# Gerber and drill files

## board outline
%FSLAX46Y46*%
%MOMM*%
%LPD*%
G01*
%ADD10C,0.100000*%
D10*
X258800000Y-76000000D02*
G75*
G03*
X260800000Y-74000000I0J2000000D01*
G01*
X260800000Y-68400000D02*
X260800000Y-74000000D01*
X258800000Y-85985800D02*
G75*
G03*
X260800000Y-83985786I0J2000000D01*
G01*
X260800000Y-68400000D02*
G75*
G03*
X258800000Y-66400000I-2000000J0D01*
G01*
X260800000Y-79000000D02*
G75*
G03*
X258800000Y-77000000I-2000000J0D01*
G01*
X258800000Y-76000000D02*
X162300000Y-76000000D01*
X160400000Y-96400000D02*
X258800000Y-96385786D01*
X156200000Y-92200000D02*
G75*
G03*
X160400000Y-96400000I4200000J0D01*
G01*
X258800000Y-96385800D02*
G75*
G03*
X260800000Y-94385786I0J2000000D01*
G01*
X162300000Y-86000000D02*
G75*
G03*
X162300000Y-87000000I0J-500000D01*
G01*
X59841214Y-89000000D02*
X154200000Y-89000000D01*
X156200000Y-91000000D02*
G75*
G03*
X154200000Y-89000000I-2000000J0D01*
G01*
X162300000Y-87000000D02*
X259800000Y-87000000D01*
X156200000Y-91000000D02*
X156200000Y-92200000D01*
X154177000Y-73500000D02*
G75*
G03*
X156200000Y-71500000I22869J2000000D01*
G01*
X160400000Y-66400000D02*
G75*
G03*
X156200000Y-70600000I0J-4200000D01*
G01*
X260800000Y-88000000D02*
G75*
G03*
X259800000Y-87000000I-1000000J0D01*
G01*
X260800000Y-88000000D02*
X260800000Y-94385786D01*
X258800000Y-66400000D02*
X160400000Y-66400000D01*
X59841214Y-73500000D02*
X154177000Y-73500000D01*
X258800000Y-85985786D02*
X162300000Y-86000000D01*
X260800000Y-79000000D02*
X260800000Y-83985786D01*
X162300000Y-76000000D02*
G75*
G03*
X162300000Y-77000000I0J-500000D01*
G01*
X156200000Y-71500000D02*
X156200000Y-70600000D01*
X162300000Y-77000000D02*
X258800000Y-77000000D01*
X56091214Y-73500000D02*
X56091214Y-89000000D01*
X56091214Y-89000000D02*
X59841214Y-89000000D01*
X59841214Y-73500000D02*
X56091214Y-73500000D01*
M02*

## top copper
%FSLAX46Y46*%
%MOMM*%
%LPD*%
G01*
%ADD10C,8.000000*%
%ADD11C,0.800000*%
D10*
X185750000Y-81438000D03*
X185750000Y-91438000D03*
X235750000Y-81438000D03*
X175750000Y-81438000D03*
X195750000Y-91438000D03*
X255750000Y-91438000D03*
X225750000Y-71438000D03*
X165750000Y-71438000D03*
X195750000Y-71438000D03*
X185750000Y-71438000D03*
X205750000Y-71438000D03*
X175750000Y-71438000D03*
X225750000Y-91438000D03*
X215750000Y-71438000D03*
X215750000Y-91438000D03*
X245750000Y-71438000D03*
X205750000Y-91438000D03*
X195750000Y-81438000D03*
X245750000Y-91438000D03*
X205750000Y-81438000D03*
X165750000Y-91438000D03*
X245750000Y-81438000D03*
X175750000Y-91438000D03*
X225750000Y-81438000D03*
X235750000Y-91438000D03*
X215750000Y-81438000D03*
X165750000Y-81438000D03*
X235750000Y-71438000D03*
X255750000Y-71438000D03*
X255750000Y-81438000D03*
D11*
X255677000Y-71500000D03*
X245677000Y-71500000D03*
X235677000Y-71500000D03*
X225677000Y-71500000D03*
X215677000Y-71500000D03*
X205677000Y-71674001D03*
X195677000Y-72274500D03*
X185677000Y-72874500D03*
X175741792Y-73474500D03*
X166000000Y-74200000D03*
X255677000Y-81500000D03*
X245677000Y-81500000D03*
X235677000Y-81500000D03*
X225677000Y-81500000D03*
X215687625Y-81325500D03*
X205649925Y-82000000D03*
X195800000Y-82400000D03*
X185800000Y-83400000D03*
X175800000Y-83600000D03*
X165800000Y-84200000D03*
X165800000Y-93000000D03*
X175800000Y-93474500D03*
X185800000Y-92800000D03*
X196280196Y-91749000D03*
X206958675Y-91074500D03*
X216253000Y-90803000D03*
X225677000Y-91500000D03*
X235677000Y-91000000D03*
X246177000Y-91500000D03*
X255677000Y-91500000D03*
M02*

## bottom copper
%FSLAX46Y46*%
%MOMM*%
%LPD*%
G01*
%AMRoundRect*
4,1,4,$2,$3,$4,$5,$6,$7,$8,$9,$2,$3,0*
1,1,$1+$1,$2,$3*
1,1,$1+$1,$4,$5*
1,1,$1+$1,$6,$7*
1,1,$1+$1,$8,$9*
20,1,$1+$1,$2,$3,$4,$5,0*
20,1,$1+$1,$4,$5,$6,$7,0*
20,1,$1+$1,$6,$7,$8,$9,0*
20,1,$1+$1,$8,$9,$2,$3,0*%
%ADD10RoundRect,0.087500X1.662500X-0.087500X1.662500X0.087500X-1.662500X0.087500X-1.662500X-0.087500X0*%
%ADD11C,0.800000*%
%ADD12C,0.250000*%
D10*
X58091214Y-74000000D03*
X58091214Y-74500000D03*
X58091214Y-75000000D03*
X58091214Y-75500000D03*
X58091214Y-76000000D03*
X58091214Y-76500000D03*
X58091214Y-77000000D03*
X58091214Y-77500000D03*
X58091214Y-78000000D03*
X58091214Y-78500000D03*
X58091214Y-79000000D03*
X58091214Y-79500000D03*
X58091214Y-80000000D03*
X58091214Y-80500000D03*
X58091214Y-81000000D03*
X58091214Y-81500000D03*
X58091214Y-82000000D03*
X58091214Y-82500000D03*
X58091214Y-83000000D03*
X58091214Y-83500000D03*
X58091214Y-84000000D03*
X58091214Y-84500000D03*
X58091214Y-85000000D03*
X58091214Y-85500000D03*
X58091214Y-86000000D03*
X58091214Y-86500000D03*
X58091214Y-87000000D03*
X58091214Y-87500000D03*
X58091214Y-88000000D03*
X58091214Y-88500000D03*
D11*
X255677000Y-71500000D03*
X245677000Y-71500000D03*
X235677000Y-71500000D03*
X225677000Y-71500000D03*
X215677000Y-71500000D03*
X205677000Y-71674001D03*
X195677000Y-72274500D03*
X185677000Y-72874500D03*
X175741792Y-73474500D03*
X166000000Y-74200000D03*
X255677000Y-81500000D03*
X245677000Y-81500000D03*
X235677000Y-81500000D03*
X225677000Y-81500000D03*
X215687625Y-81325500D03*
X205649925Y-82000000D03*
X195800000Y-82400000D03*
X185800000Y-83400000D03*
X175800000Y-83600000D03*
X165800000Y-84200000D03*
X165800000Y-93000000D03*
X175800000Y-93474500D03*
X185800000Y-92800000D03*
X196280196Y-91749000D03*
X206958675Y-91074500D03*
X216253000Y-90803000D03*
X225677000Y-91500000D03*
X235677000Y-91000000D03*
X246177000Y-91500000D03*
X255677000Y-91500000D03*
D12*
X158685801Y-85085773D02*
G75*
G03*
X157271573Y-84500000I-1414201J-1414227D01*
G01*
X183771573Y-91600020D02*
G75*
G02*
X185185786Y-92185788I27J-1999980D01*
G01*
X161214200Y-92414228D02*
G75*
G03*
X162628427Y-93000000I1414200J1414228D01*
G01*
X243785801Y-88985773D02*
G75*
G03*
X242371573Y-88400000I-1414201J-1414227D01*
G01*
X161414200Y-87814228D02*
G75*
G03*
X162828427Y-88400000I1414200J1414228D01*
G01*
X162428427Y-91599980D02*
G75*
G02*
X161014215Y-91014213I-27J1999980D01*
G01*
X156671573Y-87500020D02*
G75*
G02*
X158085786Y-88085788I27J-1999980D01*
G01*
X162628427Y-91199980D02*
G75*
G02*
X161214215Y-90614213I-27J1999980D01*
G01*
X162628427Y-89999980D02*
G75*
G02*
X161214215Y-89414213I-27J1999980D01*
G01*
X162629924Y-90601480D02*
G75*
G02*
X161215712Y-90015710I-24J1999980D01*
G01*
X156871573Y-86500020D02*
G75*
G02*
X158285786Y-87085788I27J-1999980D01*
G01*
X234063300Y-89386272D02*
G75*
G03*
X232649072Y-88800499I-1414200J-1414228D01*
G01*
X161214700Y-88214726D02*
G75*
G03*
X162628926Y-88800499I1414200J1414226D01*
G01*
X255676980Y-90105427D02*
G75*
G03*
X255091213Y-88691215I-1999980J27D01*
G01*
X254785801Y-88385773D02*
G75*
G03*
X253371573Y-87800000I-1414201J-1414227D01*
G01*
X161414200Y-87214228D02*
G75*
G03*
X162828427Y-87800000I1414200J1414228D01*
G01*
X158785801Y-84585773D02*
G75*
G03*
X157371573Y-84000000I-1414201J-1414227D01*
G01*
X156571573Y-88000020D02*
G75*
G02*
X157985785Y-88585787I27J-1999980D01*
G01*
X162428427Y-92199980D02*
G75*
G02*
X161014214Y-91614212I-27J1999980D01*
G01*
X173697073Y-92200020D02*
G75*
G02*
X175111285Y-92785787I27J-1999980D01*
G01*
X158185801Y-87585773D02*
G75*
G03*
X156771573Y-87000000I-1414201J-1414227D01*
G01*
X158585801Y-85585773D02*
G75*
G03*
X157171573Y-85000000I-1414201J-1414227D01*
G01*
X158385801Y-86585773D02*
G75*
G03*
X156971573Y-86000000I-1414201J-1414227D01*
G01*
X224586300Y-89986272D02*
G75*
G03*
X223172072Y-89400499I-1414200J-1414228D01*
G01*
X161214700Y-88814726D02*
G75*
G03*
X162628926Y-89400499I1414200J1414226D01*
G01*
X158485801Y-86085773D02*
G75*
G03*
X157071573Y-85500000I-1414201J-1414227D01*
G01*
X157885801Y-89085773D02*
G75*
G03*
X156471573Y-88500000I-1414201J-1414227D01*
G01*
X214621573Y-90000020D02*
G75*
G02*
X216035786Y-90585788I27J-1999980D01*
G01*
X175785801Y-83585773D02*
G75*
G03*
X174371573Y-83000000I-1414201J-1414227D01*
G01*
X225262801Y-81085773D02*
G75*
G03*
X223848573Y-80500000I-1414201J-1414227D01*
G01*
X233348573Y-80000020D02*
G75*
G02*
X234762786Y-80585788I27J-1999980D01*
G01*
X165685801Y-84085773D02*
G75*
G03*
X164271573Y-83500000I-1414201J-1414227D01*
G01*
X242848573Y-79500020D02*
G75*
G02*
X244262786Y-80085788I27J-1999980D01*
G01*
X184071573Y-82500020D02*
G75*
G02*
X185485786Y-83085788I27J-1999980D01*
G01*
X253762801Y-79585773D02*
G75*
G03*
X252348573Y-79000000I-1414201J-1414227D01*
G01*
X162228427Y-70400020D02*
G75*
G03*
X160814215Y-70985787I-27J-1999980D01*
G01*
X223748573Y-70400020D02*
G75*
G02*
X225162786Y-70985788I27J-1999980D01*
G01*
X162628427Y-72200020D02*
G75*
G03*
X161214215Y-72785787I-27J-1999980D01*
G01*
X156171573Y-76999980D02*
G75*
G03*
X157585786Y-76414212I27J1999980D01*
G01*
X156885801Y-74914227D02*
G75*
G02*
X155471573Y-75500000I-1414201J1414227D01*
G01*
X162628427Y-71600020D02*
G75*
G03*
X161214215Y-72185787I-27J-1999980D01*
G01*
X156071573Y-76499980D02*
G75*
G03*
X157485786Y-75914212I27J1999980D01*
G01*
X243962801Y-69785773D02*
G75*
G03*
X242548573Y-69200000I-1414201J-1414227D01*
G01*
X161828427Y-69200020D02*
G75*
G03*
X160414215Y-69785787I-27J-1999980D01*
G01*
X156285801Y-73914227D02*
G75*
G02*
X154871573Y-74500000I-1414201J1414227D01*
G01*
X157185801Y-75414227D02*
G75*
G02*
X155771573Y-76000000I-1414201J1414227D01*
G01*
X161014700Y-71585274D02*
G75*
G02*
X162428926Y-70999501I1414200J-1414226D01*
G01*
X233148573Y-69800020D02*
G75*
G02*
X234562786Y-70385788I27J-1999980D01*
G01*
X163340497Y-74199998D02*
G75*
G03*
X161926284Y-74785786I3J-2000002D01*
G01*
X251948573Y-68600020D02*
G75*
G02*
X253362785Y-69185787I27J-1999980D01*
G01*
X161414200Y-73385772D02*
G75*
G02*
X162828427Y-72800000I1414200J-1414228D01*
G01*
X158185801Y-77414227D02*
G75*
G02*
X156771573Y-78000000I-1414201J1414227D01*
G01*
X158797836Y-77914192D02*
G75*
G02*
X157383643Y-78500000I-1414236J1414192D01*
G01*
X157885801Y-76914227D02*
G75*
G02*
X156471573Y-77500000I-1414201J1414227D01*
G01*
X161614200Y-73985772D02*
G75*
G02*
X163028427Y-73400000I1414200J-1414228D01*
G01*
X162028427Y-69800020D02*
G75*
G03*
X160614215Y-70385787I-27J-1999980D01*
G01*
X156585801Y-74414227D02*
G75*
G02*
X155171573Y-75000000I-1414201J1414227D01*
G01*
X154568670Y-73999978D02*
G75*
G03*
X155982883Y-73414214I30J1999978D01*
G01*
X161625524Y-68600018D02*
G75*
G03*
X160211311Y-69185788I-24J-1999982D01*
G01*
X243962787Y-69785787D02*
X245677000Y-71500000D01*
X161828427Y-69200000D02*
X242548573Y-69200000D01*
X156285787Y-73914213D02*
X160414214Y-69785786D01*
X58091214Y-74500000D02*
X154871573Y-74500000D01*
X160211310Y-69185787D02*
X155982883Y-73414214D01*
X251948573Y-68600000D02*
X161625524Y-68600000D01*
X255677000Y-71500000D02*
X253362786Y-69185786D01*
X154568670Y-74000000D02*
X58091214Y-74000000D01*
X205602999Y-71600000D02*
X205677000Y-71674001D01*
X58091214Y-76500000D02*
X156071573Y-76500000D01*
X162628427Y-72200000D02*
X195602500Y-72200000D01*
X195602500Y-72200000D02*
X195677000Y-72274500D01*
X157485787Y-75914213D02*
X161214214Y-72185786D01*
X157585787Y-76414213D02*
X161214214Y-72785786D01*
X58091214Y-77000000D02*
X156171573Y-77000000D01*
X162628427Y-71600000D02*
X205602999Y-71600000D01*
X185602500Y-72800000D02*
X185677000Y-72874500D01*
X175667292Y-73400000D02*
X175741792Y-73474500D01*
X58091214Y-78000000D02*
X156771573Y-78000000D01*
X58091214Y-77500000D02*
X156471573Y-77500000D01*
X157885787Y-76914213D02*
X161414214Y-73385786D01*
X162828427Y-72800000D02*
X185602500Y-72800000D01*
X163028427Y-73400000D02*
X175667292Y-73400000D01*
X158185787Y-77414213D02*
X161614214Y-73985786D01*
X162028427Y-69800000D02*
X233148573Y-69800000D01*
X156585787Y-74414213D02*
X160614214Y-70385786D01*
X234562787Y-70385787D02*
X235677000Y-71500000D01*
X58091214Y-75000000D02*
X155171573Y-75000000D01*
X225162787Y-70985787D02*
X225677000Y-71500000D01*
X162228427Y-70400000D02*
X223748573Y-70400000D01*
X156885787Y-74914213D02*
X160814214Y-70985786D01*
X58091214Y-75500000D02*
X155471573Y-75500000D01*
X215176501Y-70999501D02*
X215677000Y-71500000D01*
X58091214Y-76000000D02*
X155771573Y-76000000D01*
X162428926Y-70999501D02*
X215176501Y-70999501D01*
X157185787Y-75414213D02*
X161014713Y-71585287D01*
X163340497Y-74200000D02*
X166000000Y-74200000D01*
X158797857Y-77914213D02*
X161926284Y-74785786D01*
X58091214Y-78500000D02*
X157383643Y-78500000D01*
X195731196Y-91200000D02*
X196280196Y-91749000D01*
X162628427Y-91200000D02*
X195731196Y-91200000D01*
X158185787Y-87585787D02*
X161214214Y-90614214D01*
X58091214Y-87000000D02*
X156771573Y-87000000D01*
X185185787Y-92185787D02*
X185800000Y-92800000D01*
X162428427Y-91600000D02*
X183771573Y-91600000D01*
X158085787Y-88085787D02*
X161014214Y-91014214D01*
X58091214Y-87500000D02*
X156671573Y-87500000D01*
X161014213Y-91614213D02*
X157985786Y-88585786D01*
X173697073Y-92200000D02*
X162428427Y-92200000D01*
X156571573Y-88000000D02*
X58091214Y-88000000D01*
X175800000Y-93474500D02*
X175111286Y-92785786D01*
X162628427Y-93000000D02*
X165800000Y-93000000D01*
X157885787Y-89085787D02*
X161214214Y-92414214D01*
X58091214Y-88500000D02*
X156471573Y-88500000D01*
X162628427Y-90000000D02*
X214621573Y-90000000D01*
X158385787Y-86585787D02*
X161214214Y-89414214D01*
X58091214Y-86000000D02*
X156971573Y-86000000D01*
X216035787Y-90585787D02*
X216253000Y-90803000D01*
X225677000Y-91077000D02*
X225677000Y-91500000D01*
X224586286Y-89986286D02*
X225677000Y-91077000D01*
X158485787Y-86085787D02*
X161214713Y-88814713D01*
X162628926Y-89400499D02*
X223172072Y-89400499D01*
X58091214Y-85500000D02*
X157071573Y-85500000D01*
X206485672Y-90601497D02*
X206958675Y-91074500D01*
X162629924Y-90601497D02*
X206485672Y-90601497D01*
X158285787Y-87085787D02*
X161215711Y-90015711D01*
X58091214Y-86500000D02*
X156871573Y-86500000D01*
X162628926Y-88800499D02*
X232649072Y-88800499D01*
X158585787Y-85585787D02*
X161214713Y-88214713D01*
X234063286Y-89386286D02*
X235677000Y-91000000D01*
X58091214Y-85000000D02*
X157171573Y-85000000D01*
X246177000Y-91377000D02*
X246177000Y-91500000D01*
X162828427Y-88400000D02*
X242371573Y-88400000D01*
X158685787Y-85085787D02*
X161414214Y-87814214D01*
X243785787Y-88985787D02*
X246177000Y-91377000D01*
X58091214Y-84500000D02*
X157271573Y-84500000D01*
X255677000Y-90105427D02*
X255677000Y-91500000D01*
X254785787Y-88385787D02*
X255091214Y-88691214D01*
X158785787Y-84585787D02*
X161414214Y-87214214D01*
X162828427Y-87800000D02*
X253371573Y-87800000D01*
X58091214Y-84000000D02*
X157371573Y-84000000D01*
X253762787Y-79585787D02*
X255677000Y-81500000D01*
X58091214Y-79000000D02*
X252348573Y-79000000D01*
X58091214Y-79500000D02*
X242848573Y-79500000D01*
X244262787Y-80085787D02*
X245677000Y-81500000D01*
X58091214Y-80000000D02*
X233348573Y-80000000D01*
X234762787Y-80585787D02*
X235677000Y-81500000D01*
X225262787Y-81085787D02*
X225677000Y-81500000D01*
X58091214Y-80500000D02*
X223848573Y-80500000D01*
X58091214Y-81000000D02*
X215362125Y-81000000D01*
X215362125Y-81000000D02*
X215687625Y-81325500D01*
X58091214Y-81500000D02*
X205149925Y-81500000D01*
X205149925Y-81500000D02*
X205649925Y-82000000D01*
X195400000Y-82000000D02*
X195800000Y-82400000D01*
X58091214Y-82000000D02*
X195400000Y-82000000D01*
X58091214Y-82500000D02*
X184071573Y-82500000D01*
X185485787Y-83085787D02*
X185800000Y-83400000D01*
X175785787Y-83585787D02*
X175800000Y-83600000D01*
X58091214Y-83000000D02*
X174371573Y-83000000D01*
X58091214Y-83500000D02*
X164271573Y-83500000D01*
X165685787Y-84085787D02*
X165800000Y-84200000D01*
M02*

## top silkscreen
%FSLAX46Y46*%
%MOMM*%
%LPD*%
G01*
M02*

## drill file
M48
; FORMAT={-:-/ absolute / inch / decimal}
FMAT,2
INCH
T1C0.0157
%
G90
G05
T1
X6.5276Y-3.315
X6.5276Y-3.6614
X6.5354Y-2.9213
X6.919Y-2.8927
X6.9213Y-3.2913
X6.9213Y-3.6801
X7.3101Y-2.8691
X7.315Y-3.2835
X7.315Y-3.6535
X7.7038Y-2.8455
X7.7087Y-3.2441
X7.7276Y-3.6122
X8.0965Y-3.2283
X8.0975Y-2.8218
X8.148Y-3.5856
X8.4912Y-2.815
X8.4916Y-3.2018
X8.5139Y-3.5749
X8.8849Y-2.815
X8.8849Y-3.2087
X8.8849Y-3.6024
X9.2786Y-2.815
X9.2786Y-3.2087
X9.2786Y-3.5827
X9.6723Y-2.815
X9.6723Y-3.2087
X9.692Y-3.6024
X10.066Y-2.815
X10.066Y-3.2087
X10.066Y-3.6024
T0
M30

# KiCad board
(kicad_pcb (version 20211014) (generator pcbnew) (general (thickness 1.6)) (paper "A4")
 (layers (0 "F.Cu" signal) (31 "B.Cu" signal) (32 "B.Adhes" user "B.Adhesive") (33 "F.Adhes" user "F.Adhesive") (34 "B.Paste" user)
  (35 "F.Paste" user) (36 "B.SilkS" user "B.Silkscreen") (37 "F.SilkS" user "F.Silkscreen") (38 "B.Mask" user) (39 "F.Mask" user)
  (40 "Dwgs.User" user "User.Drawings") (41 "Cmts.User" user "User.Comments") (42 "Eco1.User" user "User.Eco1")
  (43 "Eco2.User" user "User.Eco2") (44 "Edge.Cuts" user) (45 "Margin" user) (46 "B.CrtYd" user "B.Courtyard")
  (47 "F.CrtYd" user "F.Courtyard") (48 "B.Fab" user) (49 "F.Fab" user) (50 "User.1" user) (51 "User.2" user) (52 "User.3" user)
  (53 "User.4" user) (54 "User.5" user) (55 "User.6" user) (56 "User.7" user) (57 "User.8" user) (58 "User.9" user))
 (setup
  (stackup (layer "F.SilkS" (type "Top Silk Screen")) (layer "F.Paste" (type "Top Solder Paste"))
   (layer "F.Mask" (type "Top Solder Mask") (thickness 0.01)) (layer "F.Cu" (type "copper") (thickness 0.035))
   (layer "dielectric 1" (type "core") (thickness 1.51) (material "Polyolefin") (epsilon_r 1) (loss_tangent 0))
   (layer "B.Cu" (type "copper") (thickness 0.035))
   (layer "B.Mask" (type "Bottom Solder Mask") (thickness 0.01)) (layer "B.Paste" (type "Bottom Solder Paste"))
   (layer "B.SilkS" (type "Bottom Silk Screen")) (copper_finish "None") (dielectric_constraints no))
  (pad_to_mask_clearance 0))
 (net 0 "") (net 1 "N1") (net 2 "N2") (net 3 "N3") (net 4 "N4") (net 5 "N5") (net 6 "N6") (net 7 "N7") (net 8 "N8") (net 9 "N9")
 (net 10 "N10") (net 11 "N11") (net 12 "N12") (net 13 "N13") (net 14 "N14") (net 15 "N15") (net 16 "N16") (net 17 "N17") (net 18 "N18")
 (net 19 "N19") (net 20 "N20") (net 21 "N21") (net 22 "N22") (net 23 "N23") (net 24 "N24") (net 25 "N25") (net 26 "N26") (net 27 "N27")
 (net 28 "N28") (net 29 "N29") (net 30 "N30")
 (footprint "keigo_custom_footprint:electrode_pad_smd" (layer "F.Cu") (at 185.75 81.438)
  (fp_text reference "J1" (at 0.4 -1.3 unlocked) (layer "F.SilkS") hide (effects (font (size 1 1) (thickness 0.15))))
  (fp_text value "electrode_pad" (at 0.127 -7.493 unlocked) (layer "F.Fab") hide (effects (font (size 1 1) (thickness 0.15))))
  (pad "" smd circle (at 0 0) (size 8 8) (layers "F.Cu" "F.Mask") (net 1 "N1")))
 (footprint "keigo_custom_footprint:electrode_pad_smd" (layer "F.Cu") (at 185.75 91.438)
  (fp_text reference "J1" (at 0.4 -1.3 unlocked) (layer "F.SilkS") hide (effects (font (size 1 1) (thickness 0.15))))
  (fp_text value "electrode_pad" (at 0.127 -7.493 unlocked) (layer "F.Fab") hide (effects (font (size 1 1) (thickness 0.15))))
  (pad "" smd circle (at 0 0) (size 8 8) (layers "F.Cu" "F.Mask") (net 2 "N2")))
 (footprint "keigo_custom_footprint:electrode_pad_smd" (layer "F.Cu") (at 235.75 81.438)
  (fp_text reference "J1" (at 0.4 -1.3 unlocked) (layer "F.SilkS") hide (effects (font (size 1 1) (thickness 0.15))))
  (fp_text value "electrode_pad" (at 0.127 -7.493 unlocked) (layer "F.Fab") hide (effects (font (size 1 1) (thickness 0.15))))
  (pad "" smd circle (at 0 0) (size 8 8) (layers "F.Cu" "F.Mask") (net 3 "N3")))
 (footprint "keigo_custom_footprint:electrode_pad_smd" (layer "F.Cu") (at 175.75 81.438)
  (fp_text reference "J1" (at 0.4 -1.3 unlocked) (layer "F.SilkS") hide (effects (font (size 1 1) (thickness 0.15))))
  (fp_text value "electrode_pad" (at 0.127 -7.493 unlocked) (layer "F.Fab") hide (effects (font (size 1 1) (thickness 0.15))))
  (pad "" smd circle (at 0 0) (size 8 8) (layers "F.Cu" "F.Mask") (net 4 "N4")))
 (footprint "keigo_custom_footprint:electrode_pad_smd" (layer "F.Cu") (at 195.75 91.438)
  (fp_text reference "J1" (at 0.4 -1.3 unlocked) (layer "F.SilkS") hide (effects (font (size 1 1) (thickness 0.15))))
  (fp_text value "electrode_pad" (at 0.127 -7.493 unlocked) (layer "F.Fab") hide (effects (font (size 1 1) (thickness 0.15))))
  (pad "" smd circle (at 0 0) (size 8 8) (layers "F.Cu" "F.Mask") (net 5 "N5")))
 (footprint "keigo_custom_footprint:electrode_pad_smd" (layer "F.Cu") (at 255.75 91.438)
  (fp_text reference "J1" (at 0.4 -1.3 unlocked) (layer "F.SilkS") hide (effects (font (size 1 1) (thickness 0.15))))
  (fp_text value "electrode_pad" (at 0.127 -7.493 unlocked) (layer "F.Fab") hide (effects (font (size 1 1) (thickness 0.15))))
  (pad "21" smd circle (at 0 0) (size 8 8) (layers "F.Cu" "F.Mask") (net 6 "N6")))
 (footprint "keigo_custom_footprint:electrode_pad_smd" (layer "F.Cu") (at 225.75 71.438)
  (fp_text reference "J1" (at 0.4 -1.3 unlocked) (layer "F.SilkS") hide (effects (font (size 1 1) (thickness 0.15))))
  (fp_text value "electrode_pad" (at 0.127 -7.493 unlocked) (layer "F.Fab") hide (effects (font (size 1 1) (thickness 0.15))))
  (pad "" smd circle (at 0 0) (size 8 8) (layers "F.Cu" "F.Mask") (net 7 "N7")))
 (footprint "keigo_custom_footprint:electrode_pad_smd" (layer "F.Cu") (at 165.75 71.438)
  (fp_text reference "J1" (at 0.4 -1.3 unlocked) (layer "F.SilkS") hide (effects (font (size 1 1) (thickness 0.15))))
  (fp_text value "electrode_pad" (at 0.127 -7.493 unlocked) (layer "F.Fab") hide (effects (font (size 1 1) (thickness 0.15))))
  (pad "10" smd circle (at 0 0) (size 8 8) (layers "F.Cu" "F.Mask") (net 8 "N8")))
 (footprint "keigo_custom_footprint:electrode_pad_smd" (layer "F.Cu") (at 195.75 71.438)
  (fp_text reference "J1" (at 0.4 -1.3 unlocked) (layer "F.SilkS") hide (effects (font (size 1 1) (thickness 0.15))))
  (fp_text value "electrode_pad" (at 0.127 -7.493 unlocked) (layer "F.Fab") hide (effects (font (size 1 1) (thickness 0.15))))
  (pad "" smd circle (at 0 0) (size 8 8) (layers "F.Cu" "F.Mask") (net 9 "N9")))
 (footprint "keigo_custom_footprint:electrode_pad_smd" (layer "F.Cu") (at 185.75 71.438)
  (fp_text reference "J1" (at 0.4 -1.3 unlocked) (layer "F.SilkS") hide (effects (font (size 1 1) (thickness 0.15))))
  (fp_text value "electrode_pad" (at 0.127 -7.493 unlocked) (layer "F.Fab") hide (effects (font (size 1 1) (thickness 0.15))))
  (pad "" smd circle (at 0 0) (size 8 8) (layers "F.Cu" "F.Mask") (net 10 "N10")))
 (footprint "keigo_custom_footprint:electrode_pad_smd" (layer "F.Cu") (at 205.75 71.438)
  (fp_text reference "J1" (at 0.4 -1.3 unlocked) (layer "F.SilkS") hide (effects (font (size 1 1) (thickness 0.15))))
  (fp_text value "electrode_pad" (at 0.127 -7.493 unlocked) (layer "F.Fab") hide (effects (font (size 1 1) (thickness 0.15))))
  (pad "" smd circle (at 0 0) (size 8 8) (layers "F.Cu" "F.Mask") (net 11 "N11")))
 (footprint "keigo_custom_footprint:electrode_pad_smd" (layer "F.Cu") (at 175.75 71.438)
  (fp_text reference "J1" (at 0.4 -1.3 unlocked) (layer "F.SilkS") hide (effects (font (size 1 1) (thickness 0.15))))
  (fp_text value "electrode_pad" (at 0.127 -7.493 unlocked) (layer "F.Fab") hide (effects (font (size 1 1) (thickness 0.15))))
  (pad "9" smd circle (at 0 0) (size 8 8) (layers "F.Cu" "F.Mask") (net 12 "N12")))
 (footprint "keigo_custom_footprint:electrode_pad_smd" (layer "F.Cu") (at 225.75 91.438)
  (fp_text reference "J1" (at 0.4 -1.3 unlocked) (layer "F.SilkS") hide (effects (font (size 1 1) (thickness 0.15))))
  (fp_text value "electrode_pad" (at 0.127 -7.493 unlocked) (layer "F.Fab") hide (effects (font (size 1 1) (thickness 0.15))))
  (pad "" smd circle (at 0 0) (size 8 8) (layers "F.Cu" "F.Mask") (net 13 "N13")))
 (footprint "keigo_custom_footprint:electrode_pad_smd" (layer "F.Cu") (at 215.75 71.438)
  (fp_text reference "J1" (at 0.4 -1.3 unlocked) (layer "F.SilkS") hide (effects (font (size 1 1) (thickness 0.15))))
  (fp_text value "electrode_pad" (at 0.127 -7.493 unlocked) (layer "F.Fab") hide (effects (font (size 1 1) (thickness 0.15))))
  (pad "" smd circle (at 0 0) (size 8 8) (layers "F.Cu" "F.Mask") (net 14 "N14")))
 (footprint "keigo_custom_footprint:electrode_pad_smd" (layer "F.Cu") (at 215.75 91.438)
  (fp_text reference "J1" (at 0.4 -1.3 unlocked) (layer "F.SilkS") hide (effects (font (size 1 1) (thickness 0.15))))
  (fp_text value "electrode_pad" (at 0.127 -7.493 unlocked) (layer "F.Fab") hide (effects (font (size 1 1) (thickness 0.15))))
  (pad "" smd circle (at 0 0) (size 8 8) (layers "F.Cu" "F.Mask") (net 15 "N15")))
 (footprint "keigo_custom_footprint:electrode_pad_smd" (layer "F.Cu") (at 245.75 71.438)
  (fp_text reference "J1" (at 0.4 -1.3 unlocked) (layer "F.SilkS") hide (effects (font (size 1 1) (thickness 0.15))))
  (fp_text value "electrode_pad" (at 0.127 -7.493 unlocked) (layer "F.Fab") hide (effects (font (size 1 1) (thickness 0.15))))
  (pad "" smd circle (at 0 0) (size 8 8) (layers "F.Cu" "F.Mask") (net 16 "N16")))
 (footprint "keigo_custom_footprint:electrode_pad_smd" (layer "F.Cu") (at 205.75 91.438)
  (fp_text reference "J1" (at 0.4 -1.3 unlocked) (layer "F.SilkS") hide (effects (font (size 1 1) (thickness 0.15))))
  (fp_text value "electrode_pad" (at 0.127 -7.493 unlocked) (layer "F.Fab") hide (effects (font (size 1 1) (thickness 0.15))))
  (pad "" smd circle (at 0 0) (size 8 8) (layers "F.Cu" "F.Mask") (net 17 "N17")))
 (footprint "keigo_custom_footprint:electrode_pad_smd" (layer "F.Cu") (at 195.75 81.438)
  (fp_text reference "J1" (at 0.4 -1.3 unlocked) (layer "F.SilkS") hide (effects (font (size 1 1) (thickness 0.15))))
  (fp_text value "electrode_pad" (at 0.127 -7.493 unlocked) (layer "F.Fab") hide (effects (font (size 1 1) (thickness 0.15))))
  (pad "" smd circle (at 0 0) (size 8 8) (layers "F.Cu" "F.Mask") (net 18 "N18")))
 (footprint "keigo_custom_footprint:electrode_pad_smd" (layer "F.Cu") (at 245.75 91.438)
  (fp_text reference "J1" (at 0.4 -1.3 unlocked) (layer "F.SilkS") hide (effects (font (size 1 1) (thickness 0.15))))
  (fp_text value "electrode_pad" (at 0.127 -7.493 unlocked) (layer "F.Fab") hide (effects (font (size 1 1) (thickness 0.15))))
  (pad "" smd circle (at 0 0) (size 8 8) (layers "F.Cu" "F.Mask") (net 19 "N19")))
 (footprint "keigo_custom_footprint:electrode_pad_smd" (layer "F.Cu") (at 205.75 81.438)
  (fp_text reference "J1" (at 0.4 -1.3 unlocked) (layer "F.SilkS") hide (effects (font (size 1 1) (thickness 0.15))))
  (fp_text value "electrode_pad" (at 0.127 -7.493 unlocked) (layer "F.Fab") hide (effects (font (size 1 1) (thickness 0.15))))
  (pad "" smd circle (at 0 0) (size 8 8) (layers "F.Cu" "F.Mask") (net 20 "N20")))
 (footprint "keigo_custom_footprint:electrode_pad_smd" (layer "F.Cu") (at 165.75 91.438)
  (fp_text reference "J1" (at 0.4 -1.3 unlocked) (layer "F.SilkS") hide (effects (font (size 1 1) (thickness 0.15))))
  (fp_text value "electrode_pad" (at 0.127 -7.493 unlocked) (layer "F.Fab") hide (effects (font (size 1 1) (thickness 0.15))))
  (pad "30" smd circle (at 0 0) (size 8 8) (layers "F.Cu" "F.Mask") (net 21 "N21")))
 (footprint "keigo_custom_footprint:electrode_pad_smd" (layer "F.Cu") (at 245.75 81.438)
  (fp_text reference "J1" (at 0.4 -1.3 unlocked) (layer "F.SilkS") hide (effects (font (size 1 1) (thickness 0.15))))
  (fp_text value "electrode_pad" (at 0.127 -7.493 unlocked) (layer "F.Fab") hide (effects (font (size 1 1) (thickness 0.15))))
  (pad "" smd circle (at 0 0) (size 8 8) (layers "F.Cu" "F.Mask") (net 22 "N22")))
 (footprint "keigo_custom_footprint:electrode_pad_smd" (layer "F.Cu") (at 175.75 91.438)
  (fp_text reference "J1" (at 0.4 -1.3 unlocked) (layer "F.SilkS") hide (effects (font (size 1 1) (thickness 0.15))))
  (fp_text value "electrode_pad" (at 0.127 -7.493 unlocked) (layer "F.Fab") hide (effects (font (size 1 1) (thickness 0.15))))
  (pad "" smd circle (at 0 0) (size 8 8) (layers "F.Cu" "F.Mask") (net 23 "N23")))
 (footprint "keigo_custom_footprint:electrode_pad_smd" (layer "F.Cu") (at 225.75 81.438)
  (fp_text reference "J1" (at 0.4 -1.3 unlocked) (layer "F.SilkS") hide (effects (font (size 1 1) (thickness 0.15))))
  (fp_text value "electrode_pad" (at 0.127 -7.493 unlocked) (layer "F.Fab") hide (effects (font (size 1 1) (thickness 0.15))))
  (pad "" smd circle (at 0 0) (size 8 8) (layers "F.Cu" "F.Mask") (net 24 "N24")))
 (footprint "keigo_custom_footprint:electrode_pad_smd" (layer "F.Cu") (at 235.75 91.438)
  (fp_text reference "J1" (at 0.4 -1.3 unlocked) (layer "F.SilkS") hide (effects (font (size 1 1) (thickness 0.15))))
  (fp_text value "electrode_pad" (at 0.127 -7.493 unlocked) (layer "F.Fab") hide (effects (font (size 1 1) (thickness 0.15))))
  (pad "" smd circle (at 0 0) (size 8 8) (layers "F.Cu" "F.Mask") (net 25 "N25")))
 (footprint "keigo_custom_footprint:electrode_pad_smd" (layer "F.Cu") (at 215.75 81.438)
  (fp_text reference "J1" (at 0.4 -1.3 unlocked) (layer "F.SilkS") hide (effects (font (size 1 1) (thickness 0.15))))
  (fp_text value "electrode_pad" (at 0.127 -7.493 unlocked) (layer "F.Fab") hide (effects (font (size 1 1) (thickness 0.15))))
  (pad "" smd circle (at 0 0) (size 8 8) (layers "F.Cu" "F.Mask") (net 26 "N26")))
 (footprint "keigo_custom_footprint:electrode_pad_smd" (layer "F.Cu") (at 165.75 81.438)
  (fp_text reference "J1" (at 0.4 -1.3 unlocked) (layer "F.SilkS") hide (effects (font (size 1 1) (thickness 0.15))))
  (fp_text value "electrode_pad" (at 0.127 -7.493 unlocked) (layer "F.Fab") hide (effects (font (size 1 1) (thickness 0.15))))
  (pad "20" smd circle (at 0 0) (size 8 8) (layers "F.Cu" "F.Mask") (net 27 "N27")))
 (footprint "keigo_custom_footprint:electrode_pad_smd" (layer "F.Cu") (at 235.75 71.438)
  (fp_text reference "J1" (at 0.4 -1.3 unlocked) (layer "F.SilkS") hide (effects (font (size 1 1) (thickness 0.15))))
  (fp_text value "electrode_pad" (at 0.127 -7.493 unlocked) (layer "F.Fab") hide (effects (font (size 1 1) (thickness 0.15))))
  (pad "" smd circle (at 0 0) (size 8 8) (layers "F.Cu" "F.Mask") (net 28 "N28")))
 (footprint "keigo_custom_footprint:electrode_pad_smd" (layer "F.Cu") (at 255.75 71.438)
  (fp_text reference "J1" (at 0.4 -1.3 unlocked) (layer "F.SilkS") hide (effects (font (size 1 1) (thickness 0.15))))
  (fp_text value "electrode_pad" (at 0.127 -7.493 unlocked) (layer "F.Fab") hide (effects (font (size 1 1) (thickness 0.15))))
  (pad "1" smd circle (at 0 0) (size 8 8) (layers "F.Cu" "F.Mask") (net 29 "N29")))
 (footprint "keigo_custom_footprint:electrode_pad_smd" (layer "F.Cu") (at 255.75 81.438)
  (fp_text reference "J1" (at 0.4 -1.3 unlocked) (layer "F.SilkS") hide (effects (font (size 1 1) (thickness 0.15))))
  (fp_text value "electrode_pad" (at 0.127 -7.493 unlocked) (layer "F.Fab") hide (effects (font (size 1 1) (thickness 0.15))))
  (pad "11" smd circle (at 0 0) (size 8 8) (layers "F.Cu" "F.Mask") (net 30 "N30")))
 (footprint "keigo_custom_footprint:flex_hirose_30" (layer "B.Cu") (at 58.091214 80.75 -90)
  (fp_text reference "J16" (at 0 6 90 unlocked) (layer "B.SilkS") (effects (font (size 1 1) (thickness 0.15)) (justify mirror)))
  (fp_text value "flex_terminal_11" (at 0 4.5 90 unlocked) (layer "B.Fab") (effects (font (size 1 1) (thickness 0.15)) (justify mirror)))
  (fp_line (start -7.25 2) (end 8.25 2) (layer "Edge.Cuts") (width 0.1))
  (fp_line (start 8.25 2) (end 8.25 -1.75) (layer "Edge.Cuts") (width 0.1))
  (fp_line (start -7.25 -1.75) (end -7.25 2) (layer "Edge.Cuts") (width 0.1))
  (pad "1" smd roundrect (at -6.75 0 90) (size 0.35 3.5) (layers "B.Cu" "B.Paste" "B.Mask") (roundrect_rratio 0.25) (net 29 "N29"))
  (pad "2" smd roundrect (at -6.25 0 90) (size 0.35 3.5) (layers "B.Cu" "B.Paste" "B.Mask") (roundrect_rratio 0.25) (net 16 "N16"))
  (pad "3" smd roundrect (at -5.75 0 90) (size 0.35 3.5) (layers "B.Cu" "B.Paste" "B.Mask") (roundrect_rratio 0.25) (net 28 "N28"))
  (pad "4" smd roundrect (at -5.25 0 90) (size 0.35 3.5) (layers "B.Cu" "B.Paste" "B.Mask") (roundrect_rratio 0.25) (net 7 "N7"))
  (pad "5" smd roundrect (at -4.75 0 90) (size 0.35 3.5) (layers "B.Cu" "B.Paste" "B.Mask") (roundrect_rratio 0.25) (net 14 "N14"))
  (pad "6" smd roundrect (at -4.25 0 90) (size 0.35 3.5) (layers "B.Cu" "B.Paste" "B.Mask") (roundrect_rratio 0.25) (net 11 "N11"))
  (pad "7" smd roundrect (at -3.75 0 90) (size 0.35 3.5) (layers "B.Cu" "B.Paste" "B.Mask") (roundrect_rratio 0.25) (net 9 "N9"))
  (pad "8" smd roundrect (at -3.25 0 90) (size 0.35 3.5) (layers "B.Cu" "B.Paste" "B.Mask") (roundrect_rratio 0.25) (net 10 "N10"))
  (pad "9" smd roundrect (at -2.75 0 90) (size 0.35 3.5) (layers "B.Cu" "B.Paste" "B.Mask") (roundrect_rratio 0.25) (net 12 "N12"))
  (pad "10" smd roundrect (at -2.25 0 90) (size 0.35 3.5) (layers "B.Cu" "B.Paste" "B.Mask") (roundrect_rratio 0.25) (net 8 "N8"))
  (pad "11" smd roundrect (at -1.75 0 90) (size 0.35 3.5) (layers "B.Cu" "B.Paste" "B.Mask") (roundrect_rratio 0.25) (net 30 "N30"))
  (pad "12" smd roundrect (at -1.25 0 90) (size 0.35 3.5) (layers "B.Cu" "B.Paste" "B.Mask") (roundrect_rratio 0.25) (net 22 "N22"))
  (pad "13" smd roundrect (at -0.75 0 90) (size 0.35 3.5) (layers "B.Cu" "B.Paste" "B.Mask") (roundrect_rratio 0.25) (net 3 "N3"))
  (pad "14" smd roundrect (at -0.25 0 90) (size 0.35 3.5) (layers "B.Cu" "B.Paste" "B.Mask") (roundrect_rratio 0.25) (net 24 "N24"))
  (pad "15" smd roundrect (at 0.25 0 90) (size 0.35 3.5) (layers "B.Cu" "B.Paste" "B.Mask") (roundrect_rratio 0.25) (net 26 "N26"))
  (pad "16" smd roundrect (at 0.75 0 90) (size 0.35 3.5) (layers "B.Cu" "B.Paste" "B.Mask") (roundrect_rratio 0.25) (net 20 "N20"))
  (pad "17" smd roundrect (at 1.25 0 90) (size 0.35 3.5) (layers "B.Cu" "B.Paste" "B.Mask") (roundrect_rratio 0.25) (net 18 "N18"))
  (pad "18" smd roundrect (at 1.75 0 90) (size 0.35 3.5) (layers "B.Cu" "B.Paste" "B.Mask") (roundrect_rratio 0.25) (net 1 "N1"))
  (pad "19" smd roundrect (at 2.25 0 90) (size 0.35 3.5) (layers "B.Cu" "B.Paste" "B.Mask") (roundrect_rratio 0.25) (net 4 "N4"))
  (pad "20" smd roundrect (at 2.75 0 90) (size 0.35 3.5) (layers "B.Cu" "B.Paste" "B.Mask") (roundrect_rratio 0.25) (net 27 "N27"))
  (pad "21" smd roundrect (at 3.25 0 90) (size 0.35 3.5) (layers "B.Cu" "B.Paste" "B.Mask") (roundrect_rratio 0.25) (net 6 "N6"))
  (pad "22" smd roundrect (at 3.75 0 90) (size 0.35 3.5) (layers "B.Cu" "B.Paste" "B.Mask") (roundrect_rratio 0.25) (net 19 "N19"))
  (pad "23" smd roundrect (at 4.25 0 90) (size 0.35 3.5) (layers "B.Cu" "B.Paste" "B.Mask") (roundrect_rratio 0.25) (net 25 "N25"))
  (pad "24" smd roundrect (at 4.75 0 90) (size 0.35 3.5) (layers "B.Cu" "B.Paste" "B.Mask") (roundrect_rratio 0.25) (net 13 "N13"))
  (pad "25" smd roundrect (at 5.25 0 90) (size 0.35 3.5) (layers "B.Cu" "B.Paste" "B.Mask") (roundrect_rratio 0.25) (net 15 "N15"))
  (pad "26" smd roundrect (at 5.75 0 90) (size 0.35 3.5) (layers "B.Cu" "B.Paste" "B.Mask") (roundrect_rratio 0.25) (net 17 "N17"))
  (pad "27" smd roundrect (at 6.25 0 90) (size 0.35 3.5) (layers "B.Cu" "B.Paste" "B.Mask") (roundrect_rratio 0.25) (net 5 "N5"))
  (pad "28" smd roundrect (at 6.75 0 90) (size 0.35 3.5) (layers "B.Cu" "B.Paste" "B.Mask") (roundrect_rratio 0.25) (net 2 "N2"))
  (pad "29" smd roundrect (at 7.25 0 90) (size 0.35 3.5) (layers "B.Cu" "B.Paste" "B.Mask") (roundrect_rratio 0.25) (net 23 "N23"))
  (pad "30" smd roundrect (at 7.75 0 90) (size 0.35 3.5) (layers "B.Cu" "B.Paste" "B.Mask") (roundrect_rratio 0.25) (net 21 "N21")))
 (gr_arc (start 260.8 74) (mid 260.214214 75.414214) (end 258.8 76) (layer "Edge.Cuts") (width 0.1))
 (gr_line (start 260.8 68.4) (end 260.8 74) (layer "Edge.Cuts") (width 0.1))
 (gr_arc (start 260.8 83.985786) (mid 260.214214 85.4) (end 258.8 85.985786) (layer "Edge.Cuts") (width 0.1))
 (gr_arc (start 258.8 66.4) (mid 260.214214 66.985786) (end 260.8 68.4) (layer "Edge.Cuts") (width 0.1))
 (gr_arc (start 258.8 77) (mid 260.214214 77.585786) (end 260.8 79) (layer "Edge.Cuts") (width 0.1))
 (gr_line (start 258.8 76) (end 162.3 76) (layer "Edge.Cuts") (width 0.1))
 (gr_line (start 160.4 96.4) (end 258.8 96.385786) (layer "Edge.Cuts") (width 0.1))
 (gr_arc (start 160.4 96.4) (mid 157.430152 95.169848) (end 156.2 92.2) (layer "Edge.Cuts") (width 0.1))
 (gr_arc (start 260.8 94.385786) (mid 260.214214 95.8) (end 258.8 96.385786) (layer "Edge.Cuts") (width 0.1))
 (gr_arc (start 162.3 87) (mid 161.8 86.5) (end 162.3 86) (layer "Edge.Cuts") (width 0.1))
 (gr_line (start 59.841214 89) (end 154.2 89) (layer "Edge.Cuts") (width 0.1))
 (gr_arc (start 154.2 89) (mid 155.614214 89.585786) (end 156.2 91) (layer "Edge.Cuts") (width 0.1))
 (gr_line (start 162.3 87) (end 259.8 87) (layer "Edge.Cuts") (width 0.1))
 (gr_line (start 156.2 91) (end 156.2 92.2) (layer "Edge.Cuts") (width 0.1))
 (gr_arc (start 156.2 71.5) (mid 155.606067 72.922369) (end 154.177 73.5) (layer "Edge.Cuts") (width 0.1))
 (gr_arc (start 156.2 70.6) (mid 157.430152 67.630152) (end 160.4 66.4) (layer "Edge.Cuts") (width 0.1))
 (gr_arc (start 259.8 87) (mid 260.507107 87.292893) (end 260.8 88) (layer "Edge.Cuts") (width 0.1))
 (gr_line (start 260.8 88) (end 260.8 94.385786) (layer "Edge.Cuts") (width 0.1))
 (gr_line (start 258.8 66.4) (end 160.4 66.4) (layer "Edge.Cuts") (width 0.1))
 (gr_line (start 59.841214 73.5) (end 154.177 73.5) (layer "Edge.Cuts") (width 0.1))
 (gr_line (start 258.8 85.985786) (end 162.3 86) (layer "Edge.Cuts") (width 0.1))
 (gr_line (start 260.8 79) (end 260.8 83.985786) (layer "Edge.Cuts") (width 0.1))
 (gr_arc (start 162.3 77) (mid 161.8 76.5) (end 162.3 76) (layer "Edge.Cuts") (width 0.1))
 (gr_line (start 156.2 71.5) (end 156.2 70.6) (layer "Edge.Cuts") (width 0.1))
 (gr_line (start 162.3 77) (end 258.8 77) (layer "Edge.Cuts") (width 0.1))
 (via (at 255.677 71.5) (size 0.8) (drill 0.4) (layers "F.Cu" "B.Cu") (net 29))
 (segment (start 251.948573 68.6) (end 161.625524 68.6) (width 0.25) (layer "B.Cu") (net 29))
 (segment (start 160.21131 69.185787) (end 155.982883 73.414214) (width 0.25) (layer "B.Cu") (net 29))
 (segment (start 255.677 71.5) (end 253.362786 69.185786) (width 0.25) (layer "B.Cu") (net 29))
 (segment (start 154.56867 74) (end 58.091214 74) (width 0.25) (layer "B.Cu") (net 29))
 (arc (start 253.362786 69.185786) (mid 252.71394 68.752241) (end 251.948573 68.6) (width 0.25) (layer "B.Cu") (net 29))
 (arc (start 155.982883 73.414214) (mid 155.334037 73.847759) (end 154.56867 74) (width 0.25) (layer "B.Cu") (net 29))
 (arc (start 160.21131 69.185787) (mid 160.860157 68.752241) (end 161.625524 68.6) (width 0.25) (layer "B.Cu") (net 29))
 (via (at 245.677 71.5) (size 0.8) (drill 0.4) (layers "F.Cu" "B.Cu") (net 16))
 (segment (start 58.091214 74.5) (end 154.871573 74.5) (width 0.25) (layer "B.Cu") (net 16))
 (segment (start 161.828427 69.2) (end 242.548573 69.2) (width 0.25) (layer "B.Cu") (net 16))
 (segment (start 156.285787 73.914213) (end 160.414214 69.785786) (width 0.25) (layer "B.Cu") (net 16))
 (segment (start 243.962787 69.785787) (end 245.677 71.5) (width 0.25) (layer "B.Cu") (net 16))
 (arc (start 154.871573 74.5) (mid 155.63694 74.347759) (end 156.285787 73.914213) (width 0.25) (layer "B.Cu") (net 16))
 (arc (start 242.548573 69.2) (mid 243.31394 69.352241) (end 243.962787 69.785787) (width 0.25) (layer "B.Cu") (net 16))
 (arc (start 160.414214 69.785786) (mid 161.06306 69.352241) (end 161.828427 69.2) (width 0.25) (layer "B.Cu") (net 16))
 (via (at 235.677 71.5) (size 0.8) (drill 0.4) (layers "F.Cu" "B.Cu") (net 28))
 (segment (start 156.585787 74.414213) (end 160.614214 70.385786) (width 0.25) (layer "B.Cu") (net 28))
 (segment (start 162.028427 69.8) (end 233.148573 69.8) (width 0.25) (layer "B.Cu") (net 28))
 (segment (start 58.091214 75) (end 155.171573 75) (width 0.25) (layer "B.Cu") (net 28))
 (segment (start 234.562787 70.385787) (end 235.677 71.5) (width 0.25) (layer "B.Cu") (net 28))
 (arc (start 155.171573 75) (mid 155.93694 74.847759) (end 156.585787 74.414213) (width 0.25) (layer "B.Cu") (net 28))
 (arc (start 234.562787 70.385787) (mid 233.91394 69.952241) (end 233.148573 69.8) (width 0.25) (layer "B.Cu") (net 28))
 (arc (start 160.614214 70.385786) (mid 161.26306 69.952241) (end 162.028427 69.8) (width 0.25) (layer "B.Cu") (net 28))
 (via (at 225.677 71.5) (size 0.8) (drill 0.4) (layers "F.Cu" "B.Cu") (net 7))
 (segment (start 162.228427 70.4) (end 223.748573 70.4) (width 0.25) (layer "B.Cu") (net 7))
 (segment (start 58.091214 75.5) (end 155.471573 75.5) (width 0.25) (layer "B.Cu") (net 7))
 (segment (start 225.162787 70.985787) (end 225.677 71.5) (width 0.25) (layer "B.Cu") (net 7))
 (segment (start 156.885787 74.914213) (end 160.814214 70.985786) (width 0.25) (layer "B.Cu") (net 7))
 (arc (start 225.162787 70.985787) (mid 224.51394 70.552241) (end 223.748573 70.4) (width 0.25) (layer "B.Cu") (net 7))
 (arc (start 160.814214 70.985786) (mid 161.46306 70.552241) (end 162.228427 70.4) (width 0.25) (layer "B.Cu") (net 7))
 (arc (start 155.471573 75.5) (mid 156.23694 75.347759) (end 156.885787 74.914213) (width 0.25) (layer "B.Cu") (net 7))
 (via (at 215.677 71.5) (size 0.8) (drill 0.4) (layers "F.Cu" "B.Cu") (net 14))
 (segment (start 215.176501 70.999501) (end 215.677 71.5) (width 0.25) (layer "B.Cu") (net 14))
 (segment (start 58.091214 76) (end 155.771573 76) (width 0.25) (layer "B.Cu") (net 14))
 (segment (start 162.428926 70.999501) (end 215.176501 70.999501) (width 0.25) (layer "B.Cu") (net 14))
 (segment (start 157.185787 75.414213) (end 161.014713 71.585287) (width 0.25) (layer "B.Cu") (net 14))
 (arc (start 155.771573 76) (mid 156.53694 75.847759) (end 157.185787 75.414213) (width 0.25) (layer "B.Cu") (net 14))
 (arc (start 162.428926 70.999501) (mid 161.663559 71.151742) (end 161.014713 71.585287) (width 0.25) (layer "B.Cu") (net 14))
 (via (at 205.677 71.674001) (size 0.8) (drill 0.4) (layers "F.Cu" "B.Cu") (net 11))
 (segment (start 157.485787 75.914213) (end 161.214214 72.185786) (width 0.25) (layer "B.Cu") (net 11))
 (segment (start 162.628427 71.6) (end 205.602999 71.6) (width 0.25) (layer "B.Cu") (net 11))
 (segment (start 58.091214 76.5) (end 156.071573 76.5) (width 0.25) (layer "B.Cu") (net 11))
 (segment (start 205.602999 71.6) (end 205.677 71.674001) (width 0.25) (layer "B.Cu") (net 11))
 (arc (start 157.485787 75.914213) (mid 156.83694 76.347759) (end 156.071573 76.5) (width 0.25) (layer "B.Cu") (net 11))
 (arc (start 161.214214 72.185786) (mid 161.86306 71.752241) (end 162.628427 71.6) (width 0.25) (layer "B.Cu") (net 11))
 (via (at 195.677 72.2745) (size 0.8) (drill 0.4) (layers "F.Cu" "B.Cu") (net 9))
 (segment (start 157.585787 76.414213) (end 161.214214 72.785786) (width 0.25) (layer "B.Cu") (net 9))
 (segment (start 162.628427 72.2) (end 195.6025 72.2) (width 0.25) (layer "B.Cu") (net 9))
 (segment (start 58.091214 77) (end 156.171573 77) (width 0.25) (layer "B.Cu") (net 9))
 (segment (start 195.6025 72.2) (end 195.677 72.2745) (width 0.25) (layer "B.Cu") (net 9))
 (arc (start 161.214214 72.785786) (mid 161.86306 72.352241) (end 162.628427 72.2) (width 0.25) (layer "B.Cu") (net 9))
 (arc (start 157.585787 76.414213) (mid 156.93694 76.847759) (end 156.171573 77) (width 0.25) (layer "B.Cu") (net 9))
 (via (at 185.677 72.8745) (size 0.8) (drill 0.4) (layers "F.Cu" "B.Cu") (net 10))
 (segment (start 58.091214 77.5) (end 156.471573 77.5) (width 0.25) (layer "B.Cu") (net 10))
 (segment (start 157.885787 76.914213) (end 161.414214 73.385786) (width 0.25) (layer "B.Cu") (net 10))
 (segment (start 162.828427 72.8) (end 185.6025 72.8) (width 0.25) (layer "B.Cu") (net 10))
 (segment (start 185.6025 72.8) (end 185.677 72.8745) (width 0.25) (layer "B.Cu") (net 10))
 (arc (start 156.471573 77.5) (mid 157.23694 77.347759) (end 157.885787 76.914213) (width 0.25) (layer "B.Cu") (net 10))
 (arc (start 162.828427 72.8) (mid 162.06306 72.952241) (end 161.414214 73.385786) (width 0.25) (layer "B.Cu") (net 10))
 (via (at 175.741792 73.4745) (size 0.8) (drill 0.4) (layers "F.Cu" "B.Cu") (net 12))
 (segment (start 163.028427 73.4) (end 175.667292 73.4) (width 0.25) (layer "B.Cu") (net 12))
 (segment (start 158.185787 77.414213) (end 161.614214 73.985786) (width 0.25) (layer "B.Cu") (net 12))
 (segment (start 175.667292 73.4) (end 175.741792 73.4745) (width 0.25) (layer "B.Cu") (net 12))
 (segment (start 58.091214 78) (end 156.771573 78) (width 0.25) (layer "B.Cu") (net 12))
 (arc (start 163.028427 73.4) (mid 162.26306 73.552241) (end 161.614214 73.985786) (width 0.25) (layer "B.Cu") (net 12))
 (arc (start 156.771573 78) (mid 157.53694 77.847759) (end 158.185787 77.414213) (width 0.25) (layer "B.Cu") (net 12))
 (via (at 166 74.2) (size 0.8) (drill 0.4) (layers "F.Cu" "B.Cu") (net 8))
 (segment (start 158.797857 77.914213) (end 161.926284 74.785786) (width 0.25) (layer "B.Cu") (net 8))
 (segment (start 163.340497 74.2) (end 166 74.2) (width 0.25) (layer "B.Cu") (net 8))
 (segment (start 58.091214 78.5) (end 157.383643 78.5) (width 0.25) (layer "B.Cu") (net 8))
 (arc (start 161.926284 74.785786) (mid 162.57513 74.352241) (end 163.340497 74.2) (width 0.25) (layer "B.Cu") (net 8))
 (arc (start 157.383643 78.5) (mid 158.14901 78.347759) (end 158.797857 77.914213) (width 0.25) (layer "B.Cu") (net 8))
 (via (at 255.677 81.5) (size 0.8) (drill 0.4) (layers "F.Cu" "B.Cu") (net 30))
 (segment (start 253.762787 79.585787) (end 255.677 81.5) (width 0.25) (layer "B.Cu") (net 30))
 (segment (start 58.091214 79) (end 252.348573 79) (width 0.25) (layer "B.Cu") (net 30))
 (arc (start 252.348573 79) (mid 253.11394 79.152241) (end 253.762787 79.585787) (width 0.25) (layer "B.Cu") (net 30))
 (via (at 245.677 81.5) (size 0.8) (drill 0.4) (layers "F.Cu" "B.Cu") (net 22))
 (segment (start 58.091214 79.5) (end 242.848573 79.5) (width 0.25) (layer "B.Cu") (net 22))
 (segment (start 244.262787 80.085787) (end 245.677 81.5) (width 0.25) (layer "B.Cu") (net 22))
 (arc (start 244.262787 80.085787) (mid 243.61394 79.652241) (end 242.848573 79.5) (width 0.25) (layer "B.Cu") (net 22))
 (via (at 235.677 81.5) (size 0.8) (drill 0.4) (layers "F.Cu" "B.Cu") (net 3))
 (segment (start 58.091214 80) (end 233.348573 80) (width 0.25) (layer "B.Cu") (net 3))
 (segment (start 234.762787 80.585787) (end 235.677 81.5) (width 0.25) (layer "B.Cu") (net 3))
 (arc (start 234.762787 80.585787) (mid 234.11394 80.152241) (end 233.348573 80) (width 0.25) (layer "B.Cu") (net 3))
 (via (at 225.677 81.5) (size 0.8) (drill 0.4) (layers "F.Cu" "B.Cu") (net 24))
 (segment (start 225.262787 81.085787) (end 225.677 81.5) (width 0.25) (layer "B.Cu") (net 24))
 (segment (start 58.091214 80.5) (end 223.848573 80.5) (width 0.25) (layer "B.Cu") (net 24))
 (arc (start 223.848573 80.5) (mid 224.61394 80.652241) (end 225.262787 81.085787) (width 0.25) (layer "B.Cu") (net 24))
 (via (at 215.687625 81.3255) (size 0.8) (drill 0.4) (layers "F.Cu" "B.Cu") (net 26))
 (segment (start 58.091214 81) (end 215.362125 81) (width 0.25) (layer "B.Cu") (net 26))
 (segment (start 215.362125 81) (end 215.687625 81.3255) (width 0.25) (layer "B.Cu") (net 26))
 (via (at 205.649925 82) (size 0.8) (drill 0.4) (layers "F.Cu" "B.Cu") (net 20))
 (segment (start 58.091214 81.5) (end 205.149925 81.5) (width 0.25) (layer "B.Cu") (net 20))
 (segment (start 205.149925 81.5) (end 205.649925 82) (width 0.25) (layer "B.Cu") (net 20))
 (via (at 195.8 82.4) (size 0.8) (drill 0.4) (layers "F.Cu" "B.Cu") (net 18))
 (segment (start 195.4 82) (end 195.8 82.4) (width 0.25) (layer "B.Cu") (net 18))
 (segment (start 58.091214 82) (end 195.4 82) (width 0.25) (layer "B.Cu") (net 18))
 (via (at 185.8 83.4) (size 0.8) (drill 0.4) (layers "F.Cu" "B.Cu") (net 1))
 (segment (start 58.091214 82.5) (end 184.071573 82.5) (width 0.25) (layer "B.Cu") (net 1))
 (segment (start 185.485787 83.085787) (end 185.8 83.4) (width 0.25) (layer "B.Cu") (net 1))
 (arc (start 185.485787 83.085787) (mid 184.83694 82.652241) (end 184.071573 82.5) (width 0.25) (layer "B.Cu") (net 1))
 (via (at 175.8 83.6) (size 0.8) (drill 0.4) (layers "F.Cu" "B.Cu") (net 4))
 (segment (start 175.785787 83.585787) (end 175.8 83.6) (width 0.25) (layer "B.Cu") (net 4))
 (segment (start 58.091214 83) (end 174.371573 83) (width 0.25) (layer "B.Cu") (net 4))
 (arc (start 174.371573 83) (mid 175.13694 83.152241) (end 175.785787 83.585787) (width 0.25) (layer "B.Cu") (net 4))
 (via (at 165.8 84.2) (size 0.8) (drill 0.4) (layers "F.Cu" "B.Cu") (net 27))
 (segment (start 58.091214 83.5) (end 164.271573 83.5) (width 0.25) (layer "B.Cu") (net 27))
 (segment (start 165.685787 84.085787) (end 165.8 84.2) (width 0.25) (layer "B.Cu") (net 27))
 (arc (start 164.271573 83.5) (mid 165.03694 83.652241) (end 165.685787 84.085787) (width 0.25) (layer "B.Cu") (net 27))
 (via (at 255.677 91.5) (size 0.8) (drill 0.4) (layers "F.Cu" "B.Cu") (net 6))
 (segment (start 158.785787 84.585787) (end 161.414214 87.214214) (width 0.25) (layer "B.Cu") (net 6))
 (segment (start 58.091214 84) (end 157.371573 84) (width 0.25) (layer "B.Cu") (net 6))
 (segment (start 254.785787 88.385787) (end 255.091214 88.691214) (width 0.25) (layer "B.Cu") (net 6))
 (segment (start 255.677 90.105427) (end 255.677 91.5) (width 0.25) (layer "B.Cu") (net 6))
 (segment (start 162.828427 87.8) (end 253.371573 87.8) (width 0.25) (layer "B.Cu") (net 6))
 (arc (start 255.091214 88.691214) (mid 255.524759 89.34006) (end 255.677 90.105427) (width 0.25) (layer "B.Cu") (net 6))
 (arc (start 253.371573 87.8) (mid 254.13694 87.952241) (end 254.785787 88.385787) (width 0.25) (layer "B.Cu") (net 6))
 (arc (start 157.371573 84) (mid 158.13694 84.152241) (end 158.785787 84.585787) (width 0.25) (layer "B.Cu") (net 6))
 (arc (start 162.828427 87.8) (mid 162.06306 87.647759) (end 161.414214 87.214214) (width 0.25) (layer "B.Cu") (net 6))
 (via (at 246.177 91.5) (size 0.8) (drill 0.4) (layers "F.Cu" "B.Cu") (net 19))
 (segment (start 58.091214 84.5) (end 157.271573 84.5) (width 0.25) (layer "B.Cu") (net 19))
 (segment (start 158.685787 85.085787) (end 161.414214 87.814214) (width 0.25) (layer "B.Cu") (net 19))
 (segment (start 162.828427 88.4) (end 242.371573 88.4) (width 0.25) (layer "B.Cu") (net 19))
 (segment (start 243.785787 88.985787) (end 246.177 91.377) (width 0.25) (layer "B.Cu") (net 19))
 (segment (start 246.177 91.377) (end 246.177 91.5) (width 0.25) (layer "B.Cu") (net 19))
 (arc (start 162.828427 88.4) (mid 162.06306 88.247759) (end 161.414214 87.814214) (width 0.25) (layer "B.Cu") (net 19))
 (arc (start 242.371573 88.4) (mid 243.13694 88.552241) (end 243.785787 88.985787) (width 0.25) (layer "B.Cu") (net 19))
 (arc (start 157.271573 84.5) (mid 158.03694 84.652241) (end 158.685787 85.085787) (width 0.25) (layer "B.Cu") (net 19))
 (via (at 235.677 91) (size 0.8) (drill 0.4) (layers "F.Cu" "B.Cu") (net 25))
 (segment (start 234.063286 89.386286) (end 235.677 91) (width 0.25) (layer "B.Cu") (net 25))
 (segment (start 58.091214 85) (end 157.171573 85) (width 0.25) (layer "B.Cu") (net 25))
 (segment (start 162.628926 88.800499) (end 232.649072 88.800499) (width 0.25) (layer "B.Cu") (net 25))
 (segment (start 158.585787 85.585787) (end 161.214713 88.214713) (width 0.25) (layer "B.Cu") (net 25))
 (arc (start 157.171573 85) (mid 157.93694 85.152241) (end 158.585787 85.585787) (width 0.25) (layer "B.Cu") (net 25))
 (arc (start 162.628926 88.800499) (mid 161.863559 88.648258) (end 161.214713 88.214713) (width 0.25) (layer "B.Cu") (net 25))
 (arc (start 232.649072 88.800499) (mid 233.414439 88.95274) (end 234.063286 89.386286) (width 0.25) (layer "B.Cu") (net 25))
 (via (at 225.677 91.5) (size 0.8) (drill 0.4) (layers "F.Cu" "B.Cu") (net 13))
 (segment (start 58.091214 85.5) (end 157.071573 85.5) (width 0.25) (layer "B.Cu") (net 13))
 (segment (start 225.677 91.077) (end 225.677 91.5) (width 0.25) (layer "B.Cu") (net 13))
 (segment (start 158.485787 86.085787) (end 161.214713 88.814713) (width 0.25) (layer "B.Cu") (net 13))
 (segment (start 162.628926 89.400499) (end 223.172072 89.400499) (width 0.25) (layer "B.Cu") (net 13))
 (segment (start 224.586286 89.986286) (end 225.677 91.077) (width 0.25) (layer "B.Cu") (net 13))
 (arc (start 157.071573 85.5) (mid 157.83694 85.652241) (end 158.485787 86.085787) (width 0.25) (layer "B.Cu") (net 13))
 (arc (start 162.628926 89.400499) (mid 161.863559 89.248258) (end 161.214713 88.814713) (width 0.25) (layer "B.Cu") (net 13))
 (arc (start 223.172072 89.400499) (mid 223.937439 89.55274) (end 224.586286 89.986286) (width 0.25) (layer "B.Cu") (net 13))
 (via (at 216.253 90.803) (size 0.8) (drill 0.4) (layers "F.Cu" "B.Cu") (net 15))
 (segment (start 216.035787 90.585787) (end 216.253 90.803) (width 0.25) (layer "B.Cu") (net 15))
 (segment (start 158.385787 86.585787) (end 161.214214 89.414214) (width 0.25) (layer "B.Cu") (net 15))
 (segment (start 58.091214 86) (end 156.971573 86) (width 0.25) (layer "B.Cu") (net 15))
 (segment (start 162.628427 90) (end 214.621573 90) (width 0.25) (layer "B.Cu") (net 15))
 (arc (start 216.035787 90.585787) (mid 215.38694 90.152241) (end 214.621573 90) (width 0.25) (layer "B.Cu") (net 15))
 (arc (start 161.214214 89.414214) (mid 161.86306 89.847759) (end 162.628427 90) (width 0.25) (layer "B.Cu") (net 15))
 (arc (start 156.971573 86) (mid 157.73694 86.152241) (end 158.385787 86.585787) (width 0.25) (layer "B.Cu") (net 15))
 (via (at 206.958675 91.0745) (size 0.8) (drill 0.4) (layers "F.Cu" "B.Cu") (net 17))
 (segment (start 162.629924 90.601497) (end 206.485672 90.601497) (width 0.25) (layer "B.Cu") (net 17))
 (segment (start 58.091214 86.5) (end 156.871573 86.5) (width 0.25) (layer "B.Cu") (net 17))
 (segment (start 158.285787 87.085787) (end 161.215711 90.015711) (width 0.25) (layer "B.Cu") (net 17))
 (segment (start 206.485672 90.601497) (end 206.958675 91.0745) (width 0.25) (layer "B.Cu") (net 17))
 (arc (start 158.285787 87.085787) (mid 157.63694 86.652241) (end 156.871573 86.5) (width 0.25) (layer "B.Cu") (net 17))
 (arc (start 161.215711 90.015711) (mid 161.864557 90.449256) (end 162.629924 90.601497) (width 0.25) (layer "B.Cu") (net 17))
 (via (at 196.280196 91.749) (size 0.8) (drill 0.4) (layers "F.Cu" "B.Cu") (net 5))
 (segment (start 195.731196 91.2) (end 196.280196 91.749) (width 0.25) (layer "B.Cu") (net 5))
 (segment (start 158.185787 87.585787) (end 161.214214 90.614214) (width 0.25) (layer "B.Cu") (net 5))
 (segment (start 58.091214 87) (end 156.771573 87) (width 0.25) (layer "B.Cu") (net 5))
 (segment (start 162.628427 91.2) (end 195.731196 91.2) (width 0.25) (layer "B.Cu") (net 5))
 (arc (start 156.771573 87) (mid 157.53694 87.152241) (end 158.185787 87.585787) (width 0.25) (layer "B.Cu") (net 5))
 (arc (start 161.214214 90.614214) (mid 161.86306 91.047759) (end 162.628427 91.2) (width 0.25) (layer "B.Cu") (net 5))
 (via (at 185.8 92.8) (size 0.8) (drill 0.4) (layers "F.Cu" "B.Cu") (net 2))
 (segment (start 185.185787 92.185787) (end 185.8 92.8) (width 0.25) (layer "B.Cu") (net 2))
 (segment (start 158.085787 88.085787) (end 161.014214 91.014214) (width 0.25) (layer "B.Cu") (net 2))
 (segment (start 162.428427 91.6) (end 183.771573 91.6) (width 0.25) (layer "B.Cu") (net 2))
 (segment (start 58.091214 87.5) (end 156.671573 87.5) (width 0.25) (layer "B.Cu") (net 2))
 (arc (start 161.014214 91.014214) (mid 161.66306 91.447759) (end 162.428427 91.6) (width 0.25) (layer "B.Cu") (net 2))
 (arc (start 158.085787 88.085787) (mid 157.43694 87.652241) (end 156.671573 87.5) (width 0.25) (layer "B.Cu") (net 2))
 (arc (start 185.185787 92.185787) (mid 184.53694 91.752241) (end 183.771573 91.6) (width 0.25) (layer "B.Cu") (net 2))
 (via (at 175.8 93.4745) (size 0.8) (drill 0.4) (layers "F.Cu" "B.Cu") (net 23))
 (segment (start 161.014213 91.614213) (end 157.985786 88.585786) (width 0.25) (layer "B.Cu") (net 23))
 (segment (start 175.8 93.4745) (end 175.111286 92.785786) (width 0.25) (layer "B.Cu") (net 23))
 (segment (start 156.571573 88) (end 58.091214 88) (width 0.25) (layer "B.Cu") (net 23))
 (segment (start 173.697073 92.2) (end 162.428427 92.2) (width 0.25) (layer "B.Cu") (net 23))
 (arc (start 175.111286 92.785786) (mid 174.46244 92.352241) (end 173.697073 92.2) (width 0.25) (layer "B.Cu") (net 23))
 (arc (start 161.014213 91.614213) (mid 161.66306 92.047759) (end 162.428427 92.2) (width 0.25) (layer "B.Cu") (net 23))
 (arc (start 157.985786 88.585786) (mid 157.33694 88.152241) (end 156.571573 88) (width 0.25) (layer "B.Cu") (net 23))
 (via (at 165.8 93) (size 0.8) (drill 0.4) (layers "F.Cu" "B.Cu") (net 21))
 (segment (start 58.091214 88.5) (end 156.471573 88.5) (width 0.25) (layer "B.Cu") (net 21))
 (segment (start 157.885787 89.085787) (end 161.214214 92.414214) (width 0.25) (layer "B.Cu") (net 21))
 (segment (start 162.628427 93) (end 165.8 93) (width 0.25) (layer "B.Cu") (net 21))
 (arc (start 156.471573 88.5) (mid 157.23694 88.652241) (end 157.885787 89.085787) (width 0.25) (layer "B.Cu") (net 21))
 (arc (start 162.628427 93) (mid 161.86306 92.847759) (end 161.214214 92.414214) (width 0.25) (layer "B.Cu") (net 21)))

